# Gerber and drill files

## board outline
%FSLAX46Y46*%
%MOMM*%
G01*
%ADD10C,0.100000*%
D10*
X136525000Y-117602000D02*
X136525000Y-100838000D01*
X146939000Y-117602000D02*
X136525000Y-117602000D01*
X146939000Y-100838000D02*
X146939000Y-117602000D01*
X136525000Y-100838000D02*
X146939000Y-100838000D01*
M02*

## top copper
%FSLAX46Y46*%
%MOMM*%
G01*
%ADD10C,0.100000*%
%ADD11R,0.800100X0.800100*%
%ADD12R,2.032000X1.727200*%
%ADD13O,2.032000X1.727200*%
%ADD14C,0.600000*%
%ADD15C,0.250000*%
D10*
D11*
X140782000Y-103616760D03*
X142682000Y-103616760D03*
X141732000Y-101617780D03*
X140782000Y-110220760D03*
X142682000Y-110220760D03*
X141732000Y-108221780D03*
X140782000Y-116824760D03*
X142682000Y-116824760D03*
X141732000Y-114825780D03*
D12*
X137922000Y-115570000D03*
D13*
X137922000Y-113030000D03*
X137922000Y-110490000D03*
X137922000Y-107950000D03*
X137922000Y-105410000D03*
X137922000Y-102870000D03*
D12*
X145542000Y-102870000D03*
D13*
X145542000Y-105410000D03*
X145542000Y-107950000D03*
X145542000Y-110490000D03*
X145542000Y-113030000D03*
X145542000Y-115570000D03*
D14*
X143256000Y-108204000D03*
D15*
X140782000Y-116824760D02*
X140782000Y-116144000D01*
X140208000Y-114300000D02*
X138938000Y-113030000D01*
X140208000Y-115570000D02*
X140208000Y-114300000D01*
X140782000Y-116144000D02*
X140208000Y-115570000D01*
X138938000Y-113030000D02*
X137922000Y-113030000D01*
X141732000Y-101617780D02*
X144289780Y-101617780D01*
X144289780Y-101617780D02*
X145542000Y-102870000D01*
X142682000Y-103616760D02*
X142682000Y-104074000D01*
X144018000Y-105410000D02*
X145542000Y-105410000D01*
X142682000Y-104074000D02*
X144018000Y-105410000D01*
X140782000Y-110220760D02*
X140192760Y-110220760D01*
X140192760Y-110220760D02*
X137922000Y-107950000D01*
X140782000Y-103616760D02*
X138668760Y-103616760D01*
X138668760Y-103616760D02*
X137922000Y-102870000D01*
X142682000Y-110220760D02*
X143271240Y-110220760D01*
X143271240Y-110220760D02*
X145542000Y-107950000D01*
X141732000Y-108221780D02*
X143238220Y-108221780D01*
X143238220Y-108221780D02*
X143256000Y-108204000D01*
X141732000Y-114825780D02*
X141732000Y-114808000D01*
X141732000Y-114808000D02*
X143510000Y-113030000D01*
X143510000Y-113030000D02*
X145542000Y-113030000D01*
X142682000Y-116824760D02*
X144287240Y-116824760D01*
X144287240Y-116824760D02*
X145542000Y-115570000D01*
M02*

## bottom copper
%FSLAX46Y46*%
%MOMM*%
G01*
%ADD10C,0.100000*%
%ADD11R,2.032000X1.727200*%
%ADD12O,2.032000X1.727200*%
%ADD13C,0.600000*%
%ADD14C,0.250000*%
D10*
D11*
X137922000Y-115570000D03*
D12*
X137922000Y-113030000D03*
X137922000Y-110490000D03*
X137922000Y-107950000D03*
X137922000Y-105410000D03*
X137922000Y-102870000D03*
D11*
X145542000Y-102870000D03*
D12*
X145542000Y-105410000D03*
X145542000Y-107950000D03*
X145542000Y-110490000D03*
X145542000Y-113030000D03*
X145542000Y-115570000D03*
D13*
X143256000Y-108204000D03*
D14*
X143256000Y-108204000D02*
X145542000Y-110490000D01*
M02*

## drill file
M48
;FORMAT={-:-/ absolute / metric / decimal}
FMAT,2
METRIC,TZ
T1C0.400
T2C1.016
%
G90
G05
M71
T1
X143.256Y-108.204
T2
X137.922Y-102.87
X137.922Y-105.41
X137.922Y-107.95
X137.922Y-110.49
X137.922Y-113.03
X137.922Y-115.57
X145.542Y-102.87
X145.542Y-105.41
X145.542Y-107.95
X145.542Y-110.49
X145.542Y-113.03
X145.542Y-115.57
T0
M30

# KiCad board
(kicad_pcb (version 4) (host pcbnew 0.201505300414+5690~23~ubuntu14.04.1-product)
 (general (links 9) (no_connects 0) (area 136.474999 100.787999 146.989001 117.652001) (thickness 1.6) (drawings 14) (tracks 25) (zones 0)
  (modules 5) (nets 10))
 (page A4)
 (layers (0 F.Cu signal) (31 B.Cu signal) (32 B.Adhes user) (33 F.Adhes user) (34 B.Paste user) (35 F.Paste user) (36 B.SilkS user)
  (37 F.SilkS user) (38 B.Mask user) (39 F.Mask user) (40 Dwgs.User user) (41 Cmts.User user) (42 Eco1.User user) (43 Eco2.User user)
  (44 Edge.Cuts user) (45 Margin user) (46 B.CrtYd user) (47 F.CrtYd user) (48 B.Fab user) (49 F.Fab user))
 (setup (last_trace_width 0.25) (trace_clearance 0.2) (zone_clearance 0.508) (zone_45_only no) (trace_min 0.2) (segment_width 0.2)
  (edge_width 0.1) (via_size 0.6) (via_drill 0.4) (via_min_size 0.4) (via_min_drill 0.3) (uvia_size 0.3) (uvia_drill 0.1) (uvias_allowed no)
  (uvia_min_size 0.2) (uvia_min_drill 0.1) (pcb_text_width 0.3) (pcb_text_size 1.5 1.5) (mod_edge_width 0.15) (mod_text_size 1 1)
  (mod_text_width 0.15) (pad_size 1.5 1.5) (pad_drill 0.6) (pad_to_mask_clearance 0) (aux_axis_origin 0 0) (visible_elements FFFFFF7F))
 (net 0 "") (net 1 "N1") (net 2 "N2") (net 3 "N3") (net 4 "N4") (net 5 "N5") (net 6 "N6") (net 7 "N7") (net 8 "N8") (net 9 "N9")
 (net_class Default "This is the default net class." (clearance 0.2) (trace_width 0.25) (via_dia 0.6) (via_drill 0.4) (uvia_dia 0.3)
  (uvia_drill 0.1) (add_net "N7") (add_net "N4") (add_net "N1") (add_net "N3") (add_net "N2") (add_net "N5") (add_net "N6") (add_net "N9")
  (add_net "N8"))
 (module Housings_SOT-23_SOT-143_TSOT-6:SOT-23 (layer F.Cu) (at 141.732 102.616)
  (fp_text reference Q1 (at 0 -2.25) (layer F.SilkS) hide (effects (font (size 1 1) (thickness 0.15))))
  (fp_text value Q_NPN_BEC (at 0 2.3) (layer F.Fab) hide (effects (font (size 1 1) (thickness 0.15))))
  (pad 1 smd rect (at -0.95 1.00076) (size 0.8001 0.8001) (layers F.Cu F.Paste F.Mask) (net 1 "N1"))
  (pad 2 smd rect (at 0.95 1.00076) (size 0.8001 0.8001) (layers F.Cu F.Paste F.Mask) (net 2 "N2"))
  (pad 3 smd rect (at 0 -0.99822) (size 0.8001 0.8001) (layers F.Cu F.Paste F.Mask) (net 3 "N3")))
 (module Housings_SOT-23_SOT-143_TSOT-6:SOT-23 (layer F.Cu) (at 141.732 109.22)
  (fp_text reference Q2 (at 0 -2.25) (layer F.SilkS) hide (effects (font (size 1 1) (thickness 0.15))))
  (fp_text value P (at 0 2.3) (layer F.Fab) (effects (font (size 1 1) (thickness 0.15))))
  (pad 1 smd rect (at -0.95 1.00076) (size 0.8001 0.8001) (layers F.Cu F.Paste F.Mask) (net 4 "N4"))
  (pad 2 smd rect (at 0.95 1.00076) (size 0.8001 0.8001) (layers F.Cu F.Paste F.Mask) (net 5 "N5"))
  (pad 3 smd rect (at 0 -0.99822) (size 0.8001 0.8001) (layers F.Cu F.Paste F.Mask) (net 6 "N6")))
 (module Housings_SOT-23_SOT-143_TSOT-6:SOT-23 (layer F.Cu) (at 141.732 115.824)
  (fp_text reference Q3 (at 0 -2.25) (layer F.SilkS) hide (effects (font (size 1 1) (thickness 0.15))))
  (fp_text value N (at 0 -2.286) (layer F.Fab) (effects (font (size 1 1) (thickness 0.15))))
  (pad 1 smd rect (at -0.95 1.00076) (size 0.8001 0.8001) (layers F.Cu F.Paste F.Mask) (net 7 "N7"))
  (pad 2 smd rect (at 0.95 1.00076) (size 0.8001 0.8001) (layers F.Cu F.Paste F.Mask) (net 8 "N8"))
  (pad 3 smd rect (at 0 -0.99822) (size 0.8001 0.8001) (layers F.Cu F.Paste F.Mask) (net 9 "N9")))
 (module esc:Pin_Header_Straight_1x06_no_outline (layer F.Cu) (at 137.922 115.57 180)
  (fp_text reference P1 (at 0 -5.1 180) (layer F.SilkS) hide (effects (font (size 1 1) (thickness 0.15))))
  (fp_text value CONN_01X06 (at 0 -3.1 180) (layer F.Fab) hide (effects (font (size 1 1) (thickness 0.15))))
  (pad 1 thru_hole rect (at 0 0 180) (size 2.032 1.7272) (drill 1.016) (layers *.Cu *.Mask F.SilkS))
  (pad 2 thru_hole oval (at 0 2.54 180) (size 2.032 1.7272) (drill 1.016) (layers *.Cu *.Mask F.SilkS) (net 7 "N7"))
  (pad 3 thru_hole oval (at 0 5.08 180) (size 2.032 1.7272) (drill 1.016) (layers *.Cu *.Mask F.SilkS))
  (pad 4 thru_hole oval (at 0 7.62 180) (size 2.032 1.7272) (drill 1.016) (layers *.Cu *.Mask F.SilkS) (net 4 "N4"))
  (pad 5 thru_hole oval (at 0 10.16 180) (size 2.032 1.7272) (drill 1.016) (layers *.Cu *.Mask F.SilkS))
  (pad 6 thru_hole oval (at 0 12.7 180) (size 2.032 1.7272) (drill 1.016) (layers *.Cu *.Mask F.SilkS) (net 1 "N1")))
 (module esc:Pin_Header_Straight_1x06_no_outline (layer F.Cu) (at 145.542 102.87)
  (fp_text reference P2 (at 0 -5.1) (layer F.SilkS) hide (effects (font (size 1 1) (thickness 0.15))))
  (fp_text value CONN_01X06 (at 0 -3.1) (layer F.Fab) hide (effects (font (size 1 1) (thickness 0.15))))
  (pad 1 thru_hole rect (at 0 0) (size 2.032 1.7272) (drill 1.016) (layers *.Cu *.Mask F.SilkS) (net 3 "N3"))
  (pad 2 thru_hole oval (at 0 2.54) (size 2.032 1.7272) (drill 1.016) (layers *.Cu *.Mask F.SilkS) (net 2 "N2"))
  (pad 3 thru_hole oval (at 0 5.08) (size 2.032 1.7272) (drill 1.016) (layers *.Cu *.Mask F.SilkS) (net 5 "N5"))
  (pad 4 thru_hole oval (at 0 7.62) (size 2.032 1.7272) (drill 1.016) (layers *.Cu *.Mask F.SilkS) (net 6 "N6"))
  (pad 5 thru_hole oval (at 0 10.16) (size 2.032 1.7272) (drill 1.016) (layers *.Cu *.Mask F.SilkS) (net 9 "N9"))
  (pad 6 thru_hole oval (at 0 12.7) (size 2.032 1.7272) (drill 1.016) (layers *.Cu *.Mask F.SilkS) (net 8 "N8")))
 (gr_line (start 136.525 117.602) (end 136.525 100.838) (angle 90) (layer Edge.Cuts) (width 0.1))
 (gr_line (start 146.939 117.602) (end 136.525 117.602) (angle 90) (layer Edge.Cuts) (width 0.1))
 (gr_line (start 146.939 100.838) (end 146.939 117.602) (angle 90) (layer Edge.Cuts) (width 0.1))
 (gr_line (start 136.525 100.838) (end 146.939 100.838) (angle 90) (layer Edge.Cuts) (width 0.1))
 (segment (start 140.782 116.82476) (end 140.782 116.144) (width 0.25) (layer F.Cu) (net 7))
 (segment (start 140.208 114.3) (end 138.938 113.03) (width 0.25) (layer F.Cu) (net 7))
 (segment (start 140.208 115.57) (end 140.208 114.3) (width 0.25) (layer F.Cu) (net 7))
 (segment (start 140.782 116.144) (end 140.208 115.57) (width 0.25) (layer F.Cu) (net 7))
 (segment (start 138.938 113.03) (end 137.922 113.03) (width 0.25) (layer F.Cu) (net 7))
 (segment (start 141.732 101.61778) (end 144.28978 101.61778) (width 0.25) (layer F.Cu) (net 3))
 (segment (start 144.28978 101.61778) (end 145.542 102.87) (width 0.25) (layer F.Cu) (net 3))
 (segment (start 142.682 103.61676) (end 142.682 104.074) (width 0.25) (layer F.Cu) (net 2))
 (segment (start 144.018 105.41) (end 145.542 105.41) (width 0.25) (layer F.Cu) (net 2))
 (segment (start 142.682 104.074) (end 144.018 105.41) (width 0.25) (layer F.Cu) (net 2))
 (segment (start 140.782 110.22076) (end 140.19276 110.22076) (width 0.25) (layer F.Cu) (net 4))
 (segment (start 140.19276 110.22076) (end 137.922 107.95) (width 0.25) (layer F.Cu) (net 4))
 (segment (start 140.782 103.61676) (end 138.66876 103.61676) (width 0.25) (layer F.Cu) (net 1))
 (segment (start 138.66876 103.61676) (end 137.922 102.87) (width 0.25) (layer F.Cu) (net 1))
 (segment (start 142.682 110.22076) (end 143.27124 110.22076) (width 0.25) (layer F.Cu) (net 5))
 (segment (start 143.27124 110.22076) (end 145.542 107.95) (width 0.25) (layer F.Cu) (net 5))
 (segment (start 141.732 108.22178) (end 143.23822 108.22178) (width 0.25) (layer F.Cu) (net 6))
 (segment (start 143.256 108.204) (end 145.542 110.49) (width 0.25) (layer B.Cu) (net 6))
 (via (at 143.256 108.204) (size 0.6) (layers F.Cu B.Cu) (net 6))
 (segment (start 143.23822 108.22178) (end 143.256 108.204) (width 0.25) (layer F.Cu) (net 6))
 (segment (start 141.732 114.82578) (end 141.732 114.808) (width 0.25) (layer F.Cu) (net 9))
 (segment (start 141.732 114.808) (end 143.51 113.03) (width 0.25) (layer F.Cu) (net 9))
 (segment (start 143.51 113.03) (end 145.542 113.03) (width 0.25) (layer F.Cu) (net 9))
 (segment (start 142.682 116.82476) (end 144.28724 116.82476) (width 0.25) (layer F.Cu) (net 8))
 (segment (start 144.28724 116.82476) (end 145.542 115.57) (width 0.25) (layer F.Cu) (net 8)))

